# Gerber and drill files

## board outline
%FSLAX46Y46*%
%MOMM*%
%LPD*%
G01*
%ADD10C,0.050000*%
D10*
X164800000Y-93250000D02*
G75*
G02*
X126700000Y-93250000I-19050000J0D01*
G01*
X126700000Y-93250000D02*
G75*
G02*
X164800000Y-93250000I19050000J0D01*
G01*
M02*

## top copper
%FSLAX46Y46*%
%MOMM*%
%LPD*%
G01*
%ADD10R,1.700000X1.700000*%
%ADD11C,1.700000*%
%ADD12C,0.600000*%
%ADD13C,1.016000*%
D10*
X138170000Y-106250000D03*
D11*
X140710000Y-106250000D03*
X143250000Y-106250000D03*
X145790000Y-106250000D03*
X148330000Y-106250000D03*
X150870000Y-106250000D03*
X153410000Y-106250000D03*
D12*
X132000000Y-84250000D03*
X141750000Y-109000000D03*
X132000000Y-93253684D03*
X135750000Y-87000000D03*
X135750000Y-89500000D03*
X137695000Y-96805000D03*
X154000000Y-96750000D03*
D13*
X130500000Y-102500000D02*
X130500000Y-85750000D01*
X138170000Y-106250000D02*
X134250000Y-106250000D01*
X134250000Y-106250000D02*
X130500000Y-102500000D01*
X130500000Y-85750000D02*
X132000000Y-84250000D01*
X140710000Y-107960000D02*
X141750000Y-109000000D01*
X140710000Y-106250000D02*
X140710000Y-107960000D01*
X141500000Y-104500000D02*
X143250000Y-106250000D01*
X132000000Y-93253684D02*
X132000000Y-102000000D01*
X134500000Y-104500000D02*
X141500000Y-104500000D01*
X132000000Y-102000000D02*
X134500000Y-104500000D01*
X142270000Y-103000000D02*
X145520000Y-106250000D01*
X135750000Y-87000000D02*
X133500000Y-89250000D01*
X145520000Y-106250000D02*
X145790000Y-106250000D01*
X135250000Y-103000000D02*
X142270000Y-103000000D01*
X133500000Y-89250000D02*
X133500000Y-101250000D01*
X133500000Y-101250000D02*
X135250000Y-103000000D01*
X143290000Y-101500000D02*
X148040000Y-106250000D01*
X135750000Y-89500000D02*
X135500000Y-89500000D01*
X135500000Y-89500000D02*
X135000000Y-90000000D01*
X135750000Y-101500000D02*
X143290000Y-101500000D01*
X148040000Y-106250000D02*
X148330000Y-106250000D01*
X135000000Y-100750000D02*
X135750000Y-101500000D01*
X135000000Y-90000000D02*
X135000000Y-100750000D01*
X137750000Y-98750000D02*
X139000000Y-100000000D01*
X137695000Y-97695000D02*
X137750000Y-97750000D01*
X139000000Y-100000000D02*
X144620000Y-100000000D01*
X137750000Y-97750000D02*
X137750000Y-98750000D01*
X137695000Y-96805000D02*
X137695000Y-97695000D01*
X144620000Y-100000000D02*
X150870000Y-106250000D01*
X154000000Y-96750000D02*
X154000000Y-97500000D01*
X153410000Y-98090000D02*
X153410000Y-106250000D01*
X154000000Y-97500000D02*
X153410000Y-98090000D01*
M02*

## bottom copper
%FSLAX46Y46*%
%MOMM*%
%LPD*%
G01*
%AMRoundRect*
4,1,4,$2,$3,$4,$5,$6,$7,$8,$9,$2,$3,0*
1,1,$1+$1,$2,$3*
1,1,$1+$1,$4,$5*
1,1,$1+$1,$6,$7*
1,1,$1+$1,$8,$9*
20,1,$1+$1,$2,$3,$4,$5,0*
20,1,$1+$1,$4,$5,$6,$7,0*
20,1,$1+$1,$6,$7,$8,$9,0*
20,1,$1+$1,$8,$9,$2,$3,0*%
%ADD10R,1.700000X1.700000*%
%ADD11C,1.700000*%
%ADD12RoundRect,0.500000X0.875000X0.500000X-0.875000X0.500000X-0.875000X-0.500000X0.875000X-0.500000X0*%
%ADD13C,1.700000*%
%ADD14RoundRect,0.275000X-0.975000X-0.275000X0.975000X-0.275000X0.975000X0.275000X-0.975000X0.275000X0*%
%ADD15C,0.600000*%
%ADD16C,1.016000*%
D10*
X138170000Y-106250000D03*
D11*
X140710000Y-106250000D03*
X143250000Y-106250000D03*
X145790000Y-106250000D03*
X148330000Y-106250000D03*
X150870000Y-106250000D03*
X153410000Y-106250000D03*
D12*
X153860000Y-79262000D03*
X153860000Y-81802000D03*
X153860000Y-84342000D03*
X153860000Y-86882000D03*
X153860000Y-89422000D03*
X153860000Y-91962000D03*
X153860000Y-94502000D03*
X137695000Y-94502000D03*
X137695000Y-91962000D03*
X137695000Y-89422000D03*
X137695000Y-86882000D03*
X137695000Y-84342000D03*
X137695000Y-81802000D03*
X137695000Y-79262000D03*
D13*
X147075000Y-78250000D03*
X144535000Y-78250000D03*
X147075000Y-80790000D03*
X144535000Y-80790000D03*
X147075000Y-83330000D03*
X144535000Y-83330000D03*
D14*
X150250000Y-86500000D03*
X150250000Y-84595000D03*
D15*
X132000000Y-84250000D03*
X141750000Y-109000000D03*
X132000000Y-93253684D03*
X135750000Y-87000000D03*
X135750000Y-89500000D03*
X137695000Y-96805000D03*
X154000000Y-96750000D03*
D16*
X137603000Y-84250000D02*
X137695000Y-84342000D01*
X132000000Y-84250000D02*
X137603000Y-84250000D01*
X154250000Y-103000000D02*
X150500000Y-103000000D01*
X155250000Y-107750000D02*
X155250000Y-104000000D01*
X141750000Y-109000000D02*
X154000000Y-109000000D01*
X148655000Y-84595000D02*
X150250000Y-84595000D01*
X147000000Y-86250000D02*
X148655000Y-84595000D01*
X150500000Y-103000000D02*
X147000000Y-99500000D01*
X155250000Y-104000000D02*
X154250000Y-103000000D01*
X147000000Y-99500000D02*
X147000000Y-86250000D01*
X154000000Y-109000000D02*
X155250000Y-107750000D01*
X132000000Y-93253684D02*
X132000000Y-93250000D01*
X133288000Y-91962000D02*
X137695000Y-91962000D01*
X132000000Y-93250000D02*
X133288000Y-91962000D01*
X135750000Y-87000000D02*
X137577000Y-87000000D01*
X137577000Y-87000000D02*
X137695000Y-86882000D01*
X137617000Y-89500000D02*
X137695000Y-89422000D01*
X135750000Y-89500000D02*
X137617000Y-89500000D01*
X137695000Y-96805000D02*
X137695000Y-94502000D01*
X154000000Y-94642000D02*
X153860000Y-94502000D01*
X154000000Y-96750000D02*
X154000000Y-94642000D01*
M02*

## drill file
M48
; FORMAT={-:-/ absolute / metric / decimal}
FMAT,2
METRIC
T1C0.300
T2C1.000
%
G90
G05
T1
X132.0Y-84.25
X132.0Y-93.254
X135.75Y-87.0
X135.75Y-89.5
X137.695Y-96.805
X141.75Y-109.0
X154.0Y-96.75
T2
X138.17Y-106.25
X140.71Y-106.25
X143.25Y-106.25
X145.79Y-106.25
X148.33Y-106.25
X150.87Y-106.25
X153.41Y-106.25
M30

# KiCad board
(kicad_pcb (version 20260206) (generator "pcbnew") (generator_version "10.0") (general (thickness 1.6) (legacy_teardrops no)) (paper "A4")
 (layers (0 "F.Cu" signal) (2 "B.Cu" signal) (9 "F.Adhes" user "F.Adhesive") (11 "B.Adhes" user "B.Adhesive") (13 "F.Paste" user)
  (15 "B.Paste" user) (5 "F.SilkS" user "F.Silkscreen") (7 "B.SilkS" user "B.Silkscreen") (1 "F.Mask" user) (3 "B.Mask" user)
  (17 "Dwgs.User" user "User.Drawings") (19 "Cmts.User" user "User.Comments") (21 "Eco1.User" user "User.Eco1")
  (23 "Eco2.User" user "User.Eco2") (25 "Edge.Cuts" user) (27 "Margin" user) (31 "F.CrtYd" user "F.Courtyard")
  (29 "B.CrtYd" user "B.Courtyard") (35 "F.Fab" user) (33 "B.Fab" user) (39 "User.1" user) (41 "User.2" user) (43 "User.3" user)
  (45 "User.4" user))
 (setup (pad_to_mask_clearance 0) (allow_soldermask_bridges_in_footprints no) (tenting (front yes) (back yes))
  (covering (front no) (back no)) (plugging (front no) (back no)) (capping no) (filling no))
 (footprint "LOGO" (layer "F.Cu") (at 139 87.75)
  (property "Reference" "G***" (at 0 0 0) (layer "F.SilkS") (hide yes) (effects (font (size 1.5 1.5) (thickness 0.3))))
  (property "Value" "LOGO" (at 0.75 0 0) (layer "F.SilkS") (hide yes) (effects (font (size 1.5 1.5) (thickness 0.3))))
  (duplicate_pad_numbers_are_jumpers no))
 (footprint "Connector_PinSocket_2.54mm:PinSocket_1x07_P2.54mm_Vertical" (layer "F.Cu") (at 138.17 106.25 90)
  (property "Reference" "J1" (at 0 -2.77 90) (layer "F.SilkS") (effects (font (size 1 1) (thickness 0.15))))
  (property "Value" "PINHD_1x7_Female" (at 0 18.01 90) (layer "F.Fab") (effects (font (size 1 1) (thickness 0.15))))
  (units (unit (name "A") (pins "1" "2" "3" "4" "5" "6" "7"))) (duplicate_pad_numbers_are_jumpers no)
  (pad "1" thru_hole rect (at 0 0 90) (size 1.7 1.7) (drill 1) (layers "*.Cu" "*.Mask") (remove_unused_layers no) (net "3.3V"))
  (pad "2" thru_hole circle (at 0 2.54 90) (size 1.7 1.7) (drill 1) (layers "*.Cu" "*.Mask") (remove_unused_layers no) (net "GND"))
  (pad "3" thru_hole circle (at 0 5.08 90) (size 1.7 1.7) (drill 1) (layers "*.Cu" "*.Mask") (remove_unused_layers no) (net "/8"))
  (pad "4" thru_hole circle (at 0 7.62 90) (size 1.7 1.7) (drill 1) (layers "*.Cu" "*.Mask") (remove_unused_layers no) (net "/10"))
  (pad "5" thru_hole circle (at 0 10.16 90) (size 1.7 1.7) (drill 1) (layers "*.Cu" "*.Mask") (remove_unused_layers no) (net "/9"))
  (pad "6" thru_hole circle (at 0 12.7 90) (size 1.7 1.7) (drill 1) (layers "*.Cu" "*.Mask") (remove_unused_layers no) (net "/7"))
  (pad "7" thru_hole circle (at 0 15.24 90) (size 1.7 1.7) (drill 1) (layers "*.Cu" "*.Mask") (remove_unused_layers no) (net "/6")))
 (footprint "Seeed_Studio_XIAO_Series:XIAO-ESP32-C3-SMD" (layer "B.Cu") (at 154.695 97.382 180)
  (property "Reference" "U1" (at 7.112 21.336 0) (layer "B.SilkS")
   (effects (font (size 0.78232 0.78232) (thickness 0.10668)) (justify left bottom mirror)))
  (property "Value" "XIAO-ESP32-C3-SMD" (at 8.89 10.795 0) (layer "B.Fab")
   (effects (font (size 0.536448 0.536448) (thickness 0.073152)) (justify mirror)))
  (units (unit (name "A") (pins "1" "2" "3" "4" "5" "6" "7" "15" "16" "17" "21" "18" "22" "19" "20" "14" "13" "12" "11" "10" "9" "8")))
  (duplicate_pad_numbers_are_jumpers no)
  (pad "1" smd roundrect (at 0.835 18.12 180) (size 2.75 2) (layers "B.Cu" "B.Mask" "B.Paste") (roundrect_rratio 0.25)
   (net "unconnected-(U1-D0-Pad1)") (solder_mask_margin 0.0508) (thermal_bridge_angle 45))
  (pad "2" smd roundrect (at 0.835 15.58 180) (size 2.75 2) (layers "B.Cu" "B.Mask" "B.Paste") (roundrect_rratio 0.25)
   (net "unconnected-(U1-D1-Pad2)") (solder_mask_margin 0.0508) (thermal_bridge_angle 45))
  (pad "3" smd roundrect (at 0.835 13.04 180) (size 2.75 2) (layers "B.Cu" "B.Mask" "B.Paste") (roundrect_rratio 0.25)
   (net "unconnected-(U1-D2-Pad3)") (solder_mask_margin 0.0508) (thermal_bridge_angle 45))
  (pad "4" smd roundrect (at 0.835 10.5 180) (size 2.75 2) (layers "B.Cu" "B.Mask" "B.Paste") (roundrect_rratio 0.25)
   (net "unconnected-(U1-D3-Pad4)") (solder_mask_margin 0.0508) (thermal_bridge_angle 45))
  (pad "5" smd roundrect (at 0.835 7.96 180) (size 2.75 2) (layers "B.Cu" "B.Mask" "B.Paste") (roundrect_rratio 0.25)
   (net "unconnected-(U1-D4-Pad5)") (solder_mask_margin 0.0508) (thermal_bridge_angle 45))
  (pad "6" smd roundrect (at 0.835 5.42 180) (size 2.75 2) (layers "B.Cu" "B.Mask" "B.Paste") (roundrect_rratio 0.25)
   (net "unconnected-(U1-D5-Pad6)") (solder_mask_margin 0.0508) (thermal_bridge_angle 45))
  (pad "7" smd roundrect (at 0.835 2.88 180) (size 2.75 2) (layers "B.Cu" "B.Mask" "B.Paste") (roundrect_rratio 0.25) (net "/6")
   (solder_mask_margin 0.0508) (thermal_bridge_angle 45))
  (pad "8" smd roundrect (at 17 2.88 180) (size 2.75 2) (layers "B.Cu" "B.Mask" "B.Paste") (roundrect_rratio 0.25) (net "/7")
   (solder_mask_margin 0.0508) (thermal_bridge_angle 45))
  (pad "9" smd roundrect (at 17 5.42 180) (size 2.75 2) (layers "B.Cu" "B.Mask" "B.Paste") (roundrect_rratio 0.25) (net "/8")
   (solder_mask_margin 0.0508) (thermal_bridge_angle 45))
  (pad "10" smd roundrect (at 17 7.96 180) (size 2.75 2) (layers "B.Cu" "B.Mask" "B.Paste") (roundrect_rratio 0.25) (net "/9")
   (solder_mask_margin 0.0508) (thermal_bridge_angle 45))
  (pad "11" smd roundrect (at 17 10.5 180) (size 2.75 2) (layers "B.Cu" "B.Mask" "B.Paste") (roundrect_rratio 0.25) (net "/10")
   (solder_mask_margin 0.0508) (thermal_bridge_angle 45))
  (pad "12" smd roundrect (at 17 13.04 180) (size 2.75 2) (layers "B.Cu" "B.Mask" "B.Paste") (roundrect_rratio 0.25) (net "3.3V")
   (solder_mask_margin 0.0508) (thermal_bridge_angle 45))
  (pad "13" smd roundrect (at 17 15.58 180) (size 2.75 2) (layers "B.Cu" "B.Mask" "B.Paste") (roundrect_rratio 0.25)
   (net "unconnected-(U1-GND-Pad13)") (solder_mask_margin 0.0508) (thermal_bridge_angle 45))
  (pad "14" smd roundrect (at 17 18.12 180) (size 2.75 2) (layers "B.Cu" "B.Mask" "B.Paste") (roundrect_rratio 0.25)
   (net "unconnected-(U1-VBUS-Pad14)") (solder_mask_margin 0.0508) (thermal_bridge_angle 45))
  (pad "15" smd circle (at 7.62 19.132 180) (size 1.7 1.7) (layers "B.Cu" "B.Mask" "B.Paste") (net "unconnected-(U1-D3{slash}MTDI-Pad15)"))
  (pad "16" smd circle (at 10.16 19.132 180) (size 1.7 1.7) (layers "B.Cu" "B.Mask" "B.Paste") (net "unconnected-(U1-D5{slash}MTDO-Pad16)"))
  (pad "17" smd circle (at 7.62 16.592 180) (size 1.7 1.7) (layers "B.Cu" "B.Mask" "B.Paste") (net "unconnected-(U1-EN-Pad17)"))
  (pad "18" smd circle (at 10.16 16.592 180) (size 1.7 1.7) (layers "B.Cu" "B.Mask" "B.Paste") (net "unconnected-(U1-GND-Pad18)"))
  (pad "19" smd circle (at 7.62 14.052 180) (size 1.7 1.7) (layers "B.Cu" "B.Mask" "B.Paste") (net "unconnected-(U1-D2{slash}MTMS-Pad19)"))
  (pad "20" smd circle (at 10.16 14.052 180) (size 1.7 1.7) (layers "B.Cu" "B.Mask" "B.Paste") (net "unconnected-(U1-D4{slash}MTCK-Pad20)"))
  (pad "21" smd roundrect (at 4.445 10.882) (size 2.5 1.1) (layers "B.Cu" "B.Mask" "B.Paste") (roundrect_rratio 0.25)
   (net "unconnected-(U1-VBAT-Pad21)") (thermal_bridge_angle 45))
  (pad "22" smd roundrect (at 4.445 12.787) (size 2.5 1.1) (layers "B.Cu" "B.Mask" "B.Paste") (roundrect_rratio 0.25) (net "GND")
   (thermal_bridge_angle 45)))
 (gr_circle (center 145.75 93.25) (end 164.8 93.25) (stroke (width 0.05) (type solid)) (fill no) (layer "Edge.Cuts"))
 (segment (start 130.5 102.5) (end 130.5 85.75) (width 1.016) (layer "F.Cu") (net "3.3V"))
 (segment (start 138.17 106.25) (end 134.25 106.25) (width 1.016) (layer "F.Cu") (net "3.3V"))
 (segment (start 134.25 106.25) (end 130.5 102.5) (width 1.016) (layer "F.Cu") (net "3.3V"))
 (segment (start 130.5 85.75) (end 132 84.25) (width 1.016) (layer "F.Cu") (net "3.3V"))
 (via (at 132 84.25) (size 0.6) (drill 0.3) (layers "F.Cu" "B.Cu") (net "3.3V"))
 (segment (start 137.603 84.25) (end 137.695 84.342) (width 1.016) (layer "B.Cu") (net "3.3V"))
 (segment (start 132 84.25) (end 137.603 84.25) (width 1.016) (layer "B.Cu") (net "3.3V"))
 (segment (start 140.71 107.96) (end 141.75 109) (width 1.016) (layer "F.Cu") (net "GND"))
 (segment (start 140.71 106.25) (end 140.71 107.96) (width 1.016) (layer "F.Cu") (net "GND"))
 (via (at 141.75 109) (size 0.6) (drill 0.3) (layers "F.Cu" "B.Cu") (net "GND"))
 (segment (start 154.25 103) (end 150.5 103) (width 1.016) (layer "B.Cu") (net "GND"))
 (segment (start 155.25 107.75) (end 155.25 104) (width 1.016) (layer "B.Cu") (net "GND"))
 (segment (start 141.75 109) (end 154 109) (width 1.016) (layer "B.Cu") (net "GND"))
 (segment (start 148.655 84.595) (end 150.25 84.595) (width 1.016) (layer "B.Cu") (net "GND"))
 (segment (start 147 86.25) (end 148.655 84.595) (width 1.016) (layer "B.Cu") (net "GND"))
 (segment (start 150.5 103) (end 147 99.5) (width 1.016) (layer "B.Cu") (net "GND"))
 (segment (start 155.25 104) (end 154.25 103) (width 1.016) (layer "B.Cu") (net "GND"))
 (segment (start 147 99.5) (end 147 86.25) (width 1.016) (layer "B.Cu") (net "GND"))
 (segment (start 154 109) (end 155.25 107.75) (width 1.016) (layer "B.Cu") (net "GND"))
 (segment (start 141.5 104.5) (end 143.25 106.25) (width 1.016) (layer "F.Cu") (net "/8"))
 (segment (start 132 93.253684) (end 132 102) (width 1.016) (layer "F.Cu") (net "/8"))
 (segment (start 134.5 104.5) (end 141.5 104.5) (width 1.016) (layer "F.Cu") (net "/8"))
 (segment (start 132 102) (end 134.5 104.5) (width 1.016) (layer "F.Cu") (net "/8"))
 (via (at 132 93.253684) (size 0.6) (drill 0.3) (layers "F.Cu" "B.Cu") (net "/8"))
 (segment (start 132 93.253684) (end 132 93.25) (width 1.016) (layer "B.Cu") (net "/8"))
 (segment (start 133.288 91.962) (end 137.695 91.962) (width 1.016) (layer "B.Cu") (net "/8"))
 (segment (start 132 93.25) (end 133.288 91.962) (width 1.016) (layer "B.Cu") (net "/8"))
 (segment (start 142.27 103) (end 145.52 106.25) (width 1.016) (layer "F.Cu") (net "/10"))
 (segment (start 135.75 87) (end 133.5 89.25) (width 1.016) (layer "F.Cu") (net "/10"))
 (segment (start 145.52 106.25) (end 145.79 106.25) (width 1.016) (layer "F.Cu") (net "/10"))
 (segment (start 135.25 103) (end 142.27 103) (width 1.016) (layer "F.Cu") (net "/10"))
 (segment (start 133.5 89.25) (end 133.5 101.25) (width 1.016) (layer "F.Cu") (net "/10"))
 (segment (start 133.5 101.25) (end 135.25 103) (width 1.016) (layer "F.Cu") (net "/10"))
 (via (at 135.75 87) (size 0.6) (drill 0.3) (layers "F.Cu" "B.Cu") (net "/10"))
 (segment (start 135.75 87) (end 137.577 87) (width 1.016) (layer "B.Cu") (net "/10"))
 (segment (start 137.577 87) (end 137.695 86.882) (width 1.016) (layer "B.Cu") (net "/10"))
 (segment (start 143.29 101.5) (end 148.04 106.25) (width 1.016) (layer "F.Cu") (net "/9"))
 (segment (start 135.75 89.5) (end 135.5 89.5) (width 1.016) (layer "F.Cu") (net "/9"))
 (segment (start 135.5 89.5) (end 135 90) (width 1.016) (layer "F.Cu") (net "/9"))
 (segment (start 135.75 101.5) (end 143.29 101.5) (width 1.016) (layer "F.Cu") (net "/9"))
 (segment (start 148.04 106.25) (end 148.33 106.25) (width 1.016) (layer "F.Cu") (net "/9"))
 (segment (start 135 100.75) (end 135.75 101.5) (width 1.016) (layer "F.Cu") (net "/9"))
 (segment (start 135 90) (end 135 100.75) (width 1.016) (layer "F.Cu") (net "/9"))
 (via (at 135.75 89.5) (size 0.6) (drill 0.3) (layers "F.Cu" "B.Cu") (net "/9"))
 (segment (start 137.617 89.5) (end 137.695 89.422) (width 1.016) (layer "B.Cu") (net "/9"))
 (segment (start 135.75 89.5) (end 137.617 89.5) (width 1.016) (layer "B.Cu") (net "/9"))
 (segment (start 137.75 98.75) (end 139 100) (width 1.016) (layer "F.Cu") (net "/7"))
 (segment (start 137.695 97.695) (end 137.75 97.75) (width 1.016) (layer "F.Cu") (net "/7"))
 (segment (start 139 100) (end 144.62 100) (width 1.016) (layer "F.Cu") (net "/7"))
 (segment (start 137.75 97.75) (end 137.75 98.75) (width 1.016) (layer "F.Cu") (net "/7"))
 (segment (start 137.695 96.805) (end 137.695 97.695) (width 1.016) (layer "F.Cu") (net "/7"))
 (segment (start 144.62 100) (end 150.87 106.25) (width 1.016) (layer "F.Cu") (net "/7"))
 (via (at 137.695 96.805) (size 0.6) (drill 0.3) (layers "F.Cu" "B.Cu") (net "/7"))
 (segment (start 137.695 96.805) (end 137.695 94.502) (width 1.016) (layer "B.Cu") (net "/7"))
 (segment (start 154 96.75) (end 154 97.5) (width 1.016) (layer "F.Cu") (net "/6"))
 (segment (start 153.41 98.09) (end 153.41 106.25) (width 1.016) (layer "F.Cu") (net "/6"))
 (segment (start 154 97.5) (end 153.41 98.09) (width 1.016) (layer "F.Cu") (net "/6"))
 (via (at 154 96.75) (size 0.6) (drill 0.3) (layers "F.Cu" "B.Cu") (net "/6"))
 (segment (start 154 94.642) (end 153.86 94.502) (width 1.016) (layer "B.Cu") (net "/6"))
 (segment (start 154 96.75) (end 154 94.642) (width 1.016) (layer "B.Cu") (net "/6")))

